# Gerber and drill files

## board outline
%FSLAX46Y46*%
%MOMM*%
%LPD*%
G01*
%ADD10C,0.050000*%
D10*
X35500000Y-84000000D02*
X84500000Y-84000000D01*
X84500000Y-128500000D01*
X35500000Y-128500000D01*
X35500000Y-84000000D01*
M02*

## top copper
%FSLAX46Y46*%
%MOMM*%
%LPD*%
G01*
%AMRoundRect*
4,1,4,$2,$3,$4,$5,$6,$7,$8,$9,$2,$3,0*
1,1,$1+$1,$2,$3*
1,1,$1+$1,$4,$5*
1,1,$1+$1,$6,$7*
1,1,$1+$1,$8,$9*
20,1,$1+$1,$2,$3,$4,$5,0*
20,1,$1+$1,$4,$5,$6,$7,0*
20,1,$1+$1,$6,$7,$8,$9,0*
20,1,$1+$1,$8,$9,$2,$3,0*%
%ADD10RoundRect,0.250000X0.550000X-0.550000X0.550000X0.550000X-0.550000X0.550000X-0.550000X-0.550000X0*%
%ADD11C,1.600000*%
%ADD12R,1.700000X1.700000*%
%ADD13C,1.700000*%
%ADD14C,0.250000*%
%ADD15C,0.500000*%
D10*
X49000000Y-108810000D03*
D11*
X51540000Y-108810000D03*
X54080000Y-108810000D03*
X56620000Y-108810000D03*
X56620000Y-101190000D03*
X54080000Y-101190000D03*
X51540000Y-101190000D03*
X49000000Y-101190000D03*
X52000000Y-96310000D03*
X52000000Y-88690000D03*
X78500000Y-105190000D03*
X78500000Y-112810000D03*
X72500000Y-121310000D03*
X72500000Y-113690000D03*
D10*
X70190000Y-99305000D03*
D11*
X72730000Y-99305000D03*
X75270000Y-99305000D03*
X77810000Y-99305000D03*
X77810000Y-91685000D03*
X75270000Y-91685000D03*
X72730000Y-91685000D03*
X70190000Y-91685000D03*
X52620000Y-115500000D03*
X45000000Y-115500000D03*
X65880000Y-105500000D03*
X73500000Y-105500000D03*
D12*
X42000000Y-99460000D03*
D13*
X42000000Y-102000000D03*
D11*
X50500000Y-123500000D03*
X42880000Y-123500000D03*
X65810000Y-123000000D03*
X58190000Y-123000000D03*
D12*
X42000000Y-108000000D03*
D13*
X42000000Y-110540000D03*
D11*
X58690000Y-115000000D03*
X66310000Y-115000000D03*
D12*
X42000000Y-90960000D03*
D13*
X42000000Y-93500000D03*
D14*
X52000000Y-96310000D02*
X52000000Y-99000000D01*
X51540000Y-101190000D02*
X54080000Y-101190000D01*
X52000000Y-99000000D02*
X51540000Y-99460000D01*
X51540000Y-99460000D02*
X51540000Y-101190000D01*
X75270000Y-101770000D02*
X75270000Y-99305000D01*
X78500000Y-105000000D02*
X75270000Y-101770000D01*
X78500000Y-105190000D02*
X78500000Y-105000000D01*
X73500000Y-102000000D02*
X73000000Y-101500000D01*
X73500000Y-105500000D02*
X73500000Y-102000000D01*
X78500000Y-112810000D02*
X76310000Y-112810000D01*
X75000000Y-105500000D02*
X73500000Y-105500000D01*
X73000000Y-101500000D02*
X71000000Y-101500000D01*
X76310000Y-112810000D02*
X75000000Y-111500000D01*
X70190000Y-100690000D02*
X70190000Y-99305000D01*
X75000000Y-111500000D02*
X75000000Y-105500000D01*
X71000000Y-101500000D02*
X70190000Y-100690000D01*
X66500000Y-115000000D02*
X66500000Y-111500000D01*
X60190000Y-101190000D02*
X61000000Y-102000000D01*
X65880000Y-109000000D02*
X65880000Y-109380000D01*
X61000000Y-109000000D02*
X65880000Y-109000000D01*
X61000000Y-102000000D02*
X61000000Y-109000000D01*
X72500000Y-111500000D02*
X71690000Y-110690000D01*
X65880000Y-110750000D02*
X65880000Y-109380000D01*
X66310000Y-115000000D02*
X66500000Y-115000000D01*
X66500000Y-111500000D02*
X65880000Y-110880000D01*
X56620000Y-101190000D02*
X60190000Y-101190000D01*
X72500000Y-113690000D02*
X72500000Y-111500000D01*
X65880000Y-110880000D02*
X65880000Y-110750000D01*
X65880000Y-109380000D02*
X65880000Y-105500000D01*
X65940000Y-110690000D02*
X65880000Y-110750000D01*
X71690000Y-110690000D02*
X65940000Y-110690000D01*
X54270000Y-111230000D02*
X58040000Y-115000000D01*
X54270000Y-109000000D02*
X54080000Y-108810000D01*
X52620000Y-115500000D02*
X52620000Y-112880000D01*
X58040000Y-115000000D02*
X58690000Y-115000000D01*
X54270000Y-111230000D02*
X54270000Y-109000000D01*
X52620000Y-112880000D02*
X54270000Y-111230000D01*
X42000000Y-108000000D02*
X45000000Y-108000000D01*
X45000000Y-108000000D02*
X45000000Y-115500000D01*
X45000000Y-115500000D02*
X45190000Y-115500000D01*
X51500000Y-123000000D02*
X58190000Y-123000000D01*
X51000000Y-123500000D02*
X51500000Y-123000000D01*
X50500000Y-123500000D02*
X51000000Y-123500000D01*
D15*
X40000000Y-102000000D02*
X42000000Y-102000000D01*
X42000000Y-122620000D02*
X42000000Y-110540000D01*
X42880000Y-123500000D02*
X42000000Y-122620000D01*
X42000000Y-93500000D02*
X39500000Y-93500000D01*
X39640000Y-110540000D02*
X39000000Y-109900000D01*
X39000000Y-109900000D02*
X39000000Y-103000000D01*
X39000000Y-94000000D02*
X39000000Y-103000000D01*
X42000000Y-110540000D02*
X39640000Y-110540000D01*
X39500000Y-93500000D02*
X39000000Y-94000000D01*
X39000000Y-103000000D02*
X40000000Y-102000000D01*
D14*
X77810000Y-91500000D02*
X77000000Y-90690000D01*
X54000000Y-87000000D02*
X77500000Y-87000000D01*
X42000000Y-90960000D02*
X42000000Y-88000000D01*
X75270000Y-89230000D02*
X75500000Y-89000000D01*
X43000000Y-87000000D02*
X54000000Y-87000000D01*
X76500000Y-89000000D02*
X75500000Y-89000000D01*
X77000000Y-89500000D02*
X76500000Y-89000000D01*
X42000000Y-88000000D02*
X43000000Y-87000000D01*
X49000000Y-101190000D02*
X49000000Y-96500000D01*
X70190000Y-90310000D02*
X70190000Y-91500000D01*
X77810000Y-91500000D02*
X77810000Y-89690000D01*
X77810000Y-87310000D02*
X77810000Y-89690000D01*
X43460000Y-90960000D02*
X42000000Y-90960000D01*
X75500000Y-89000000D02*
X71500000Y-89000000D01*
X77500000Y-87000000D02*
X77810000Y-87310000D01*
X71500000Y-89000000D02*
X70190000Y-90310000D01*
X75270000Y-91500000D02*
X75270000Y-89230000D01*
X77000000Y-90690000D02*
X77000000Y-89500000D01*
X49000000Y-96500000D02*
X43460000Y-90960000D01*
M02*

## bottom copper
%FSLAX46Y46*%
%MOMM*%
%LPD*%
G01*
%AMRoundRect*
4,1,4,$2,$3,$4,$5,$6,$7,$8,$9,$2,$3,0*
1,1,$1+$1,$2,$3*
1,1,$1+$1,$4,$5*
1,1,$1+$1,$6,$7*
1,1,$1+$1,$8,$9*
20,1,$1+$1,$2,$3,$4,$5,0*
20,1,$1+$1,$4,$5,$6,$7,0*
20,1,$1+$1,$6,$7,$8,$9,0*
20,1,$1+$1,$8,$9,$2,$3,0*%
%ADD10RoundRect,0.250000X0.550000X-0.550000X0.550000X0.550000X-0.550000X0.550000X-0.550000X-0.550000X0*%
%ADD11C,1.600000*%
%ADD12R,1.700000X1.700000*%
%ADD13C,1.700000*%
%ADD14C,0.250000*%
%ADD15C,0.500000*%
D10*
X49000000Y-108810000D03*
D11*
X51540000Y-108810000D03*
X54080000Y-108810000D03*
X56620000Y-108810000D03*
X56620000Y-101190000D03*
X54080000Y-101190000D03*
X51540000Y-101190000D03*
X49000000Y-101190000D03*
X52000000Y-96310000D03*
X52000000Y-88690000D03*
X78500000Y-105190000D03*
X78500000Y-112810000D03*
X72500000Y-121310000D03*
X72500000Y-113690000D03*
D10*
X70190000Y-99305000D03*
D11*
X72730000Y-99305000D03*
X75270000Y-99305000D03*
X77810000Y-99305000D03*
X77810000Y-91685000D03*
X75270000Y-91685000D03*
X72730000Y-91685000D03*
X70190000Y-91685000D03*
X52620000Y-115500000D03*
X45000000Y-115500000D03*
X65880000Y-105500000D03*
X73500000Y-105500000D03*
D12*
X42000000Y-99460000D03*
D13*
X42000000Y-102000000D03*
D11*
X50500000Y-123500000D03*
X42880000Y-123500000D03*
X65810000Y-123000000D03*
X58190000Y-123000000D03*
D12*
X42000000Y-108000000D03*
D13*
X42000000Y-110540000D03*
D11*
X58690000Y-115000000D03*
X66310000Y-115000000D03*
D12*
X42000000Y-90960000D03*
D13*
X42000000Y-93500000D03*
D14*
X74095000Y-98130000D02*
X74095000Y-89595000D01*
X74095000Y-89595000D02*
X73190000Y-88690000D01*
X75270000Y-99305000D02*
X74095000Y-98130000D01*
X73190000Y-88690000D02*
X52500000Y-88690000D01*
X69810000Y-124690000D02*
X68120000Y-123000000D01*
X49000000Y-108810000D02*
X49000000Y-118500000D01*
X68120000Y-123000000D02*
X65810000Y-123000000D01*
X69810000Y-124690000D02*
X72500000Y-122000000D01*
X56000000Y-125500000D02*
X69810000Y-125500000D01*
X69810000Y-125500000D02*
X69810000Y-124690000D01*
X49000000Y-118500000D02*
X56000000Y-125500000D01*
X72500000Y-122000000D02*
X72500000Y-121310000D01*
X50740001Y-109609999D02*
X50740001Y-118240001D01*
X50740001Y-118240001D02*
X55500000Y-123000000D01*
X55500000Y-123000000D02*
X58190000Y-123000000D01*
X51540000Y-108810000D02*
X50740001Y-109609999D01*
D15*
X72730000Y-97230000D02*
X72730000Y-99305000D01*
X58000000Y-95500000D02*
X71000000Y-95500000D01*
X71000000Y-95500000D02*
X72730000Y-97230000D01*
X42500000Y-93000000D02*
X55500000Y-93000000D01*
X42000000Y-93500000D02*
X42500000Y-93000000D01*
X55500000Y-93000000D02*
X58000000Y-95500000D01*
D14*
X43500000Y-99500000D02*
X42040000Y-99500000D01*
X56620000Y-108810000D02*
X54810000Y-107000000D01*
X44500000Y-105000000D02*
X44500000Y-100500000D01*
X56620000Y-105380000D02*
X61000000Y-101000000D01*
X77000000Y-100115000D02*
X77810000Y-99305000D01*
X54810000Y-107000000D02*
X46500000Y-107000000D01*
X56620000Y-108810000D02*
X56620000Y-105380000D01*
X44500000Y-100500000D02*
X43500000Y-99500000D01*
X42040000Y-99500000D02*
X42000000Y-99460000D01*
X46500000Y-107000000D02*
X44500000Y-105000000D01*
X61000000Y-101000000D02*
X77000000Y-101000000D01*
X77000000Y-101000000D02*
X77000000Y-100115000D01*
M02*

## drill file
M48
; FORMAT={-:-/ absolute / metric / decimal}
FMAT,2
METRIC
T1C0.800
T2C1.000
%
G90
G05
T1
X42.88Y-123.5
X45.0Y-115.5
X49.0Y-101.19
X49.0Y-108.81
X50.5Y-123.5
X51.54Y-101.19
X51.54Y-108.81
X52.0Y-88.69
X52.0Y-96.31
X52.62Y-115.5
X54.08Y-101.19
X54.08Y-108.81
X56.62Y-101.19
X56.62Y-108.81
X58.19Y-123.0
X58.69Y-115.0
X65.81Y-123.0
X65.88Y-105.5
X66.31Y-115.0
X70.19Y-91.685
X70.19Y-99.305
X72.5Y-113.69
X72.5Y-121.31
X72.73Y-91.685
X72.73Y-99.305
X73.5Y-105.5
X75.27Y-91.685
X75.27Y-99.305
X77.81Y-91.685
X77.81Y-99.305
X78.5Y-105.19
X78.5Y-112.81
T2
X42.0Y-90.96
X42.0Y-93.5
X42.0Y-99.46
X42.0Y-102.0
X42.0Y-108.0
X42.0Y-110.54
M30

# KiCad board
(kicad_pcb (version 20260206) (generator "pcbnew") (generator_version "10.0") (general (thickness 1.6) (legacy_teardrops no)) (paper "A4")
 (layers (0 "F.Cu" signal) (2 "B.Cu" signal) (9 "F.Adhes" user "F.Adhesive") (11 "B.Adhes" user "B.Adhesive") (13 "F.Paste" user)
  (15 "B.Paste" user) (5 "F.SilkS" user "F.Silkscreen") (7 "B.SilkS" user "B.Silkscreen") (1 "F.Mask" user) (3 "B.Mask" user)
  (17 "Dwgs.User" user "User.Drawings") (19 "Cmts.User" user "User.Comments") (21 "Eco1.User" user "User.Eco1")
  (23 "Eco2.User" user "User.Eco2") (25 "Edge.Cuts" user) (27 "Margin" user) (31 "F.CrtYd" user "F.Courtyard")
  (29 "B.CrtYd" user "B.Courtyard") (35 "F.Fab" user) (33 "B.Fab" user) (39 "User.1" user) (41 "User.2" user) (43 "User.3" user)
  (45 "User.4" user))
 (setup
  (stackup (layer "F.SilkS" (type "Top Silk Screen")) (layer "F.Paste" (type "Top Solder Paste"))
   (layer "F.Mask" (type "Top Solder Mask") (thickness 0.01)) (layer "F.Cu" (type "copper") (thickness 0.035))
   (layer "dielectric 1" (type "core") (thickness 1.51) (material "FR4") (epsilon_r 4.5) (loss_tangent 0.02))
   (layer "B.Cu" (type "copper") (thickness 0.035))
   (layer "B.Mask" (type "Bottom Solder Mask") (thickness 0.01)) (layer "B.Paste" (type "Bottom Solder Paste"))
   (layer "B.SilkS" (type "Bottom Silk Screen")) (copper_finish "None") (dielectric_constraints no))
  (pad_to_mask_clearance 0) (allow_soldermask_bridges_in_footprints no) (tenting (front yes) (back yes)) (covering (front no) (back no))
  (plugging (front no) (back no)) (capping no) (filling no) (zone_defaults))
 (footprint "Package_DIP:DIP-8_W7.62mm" (layer "F.Cu") (at 49 108.81 90)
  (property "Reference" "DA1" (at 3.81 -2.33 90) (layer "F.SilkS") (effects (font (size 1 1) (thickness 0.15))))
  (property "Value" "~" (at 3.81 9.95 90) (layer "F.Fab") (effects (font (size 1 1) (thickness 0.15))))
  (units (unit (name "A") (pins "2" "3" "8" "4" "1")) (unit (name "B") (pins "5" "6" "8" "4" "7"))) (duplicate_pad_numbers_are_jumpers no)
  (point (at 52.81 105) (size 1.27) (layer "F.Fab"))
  (pad "1" thru_hole roundrect (at 0 0 90) (size 1.6 1.6) (drill 0.8) (layers "*.Cu" "*.Mask") (remove_unused_layers no)
   (roundrect_rratio 0.15625) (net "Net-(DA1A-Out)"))
  (pad "2" thru_hole circle (at 0 2.54 90) (size 1.6 1.6) (drill 0.8) (layers "*.Cu" "*.Mask") (remove_unused_layers no)
   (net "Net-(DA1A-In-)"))
  (pad "3" thru_hole circle (at 0 5.08 90) (size 1.6 1.6) (drill 0.8) (layers "*.Cu" "*.Mask") (remove_unused_layers no)
   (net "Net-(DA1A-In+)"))
  (pad "4" thru_hole circle (at 0 7.62 90) (size 1.6 1.6) (drill 0.8) (layers "*.Cu" "*.Mask") (remove_unused_layers no) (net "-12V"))
  (pad "5" thru_hole circle (at 7.62 7.62 90) (size 1.6 1.6) (drill 0.8) (layers "*.Cu" "*.Mask") (remove_unused_layers no)
   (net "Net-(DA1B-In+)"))
  (pad "6" thru_hole circle (at 7.62 5.08 90) (size 1.6 1.6) (drill 0.8) (layers "*.Cu" "*.Mask") (remove_unused_layers no)
   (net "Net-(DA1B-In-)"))
  (pad "7" thru_hole circle (at 7.62 2.54 90) (size 1.6 1.6) (drill 0.8) (layers "*.Cu" "*.Mask") (remove_unused_layers no)
   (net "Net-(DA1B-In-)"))
  (pad "8" thru_hole circle (at 7.62 0 90) (size 1.6 1.6) (drill 0.8) (layers "*.Cu" "*.Mask") (remove_unused_layers no) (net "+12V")))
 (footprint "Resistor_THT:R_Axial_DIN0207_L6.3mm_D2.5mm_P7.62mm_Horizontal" (layer "F.Cu") (at 52 96.31 90)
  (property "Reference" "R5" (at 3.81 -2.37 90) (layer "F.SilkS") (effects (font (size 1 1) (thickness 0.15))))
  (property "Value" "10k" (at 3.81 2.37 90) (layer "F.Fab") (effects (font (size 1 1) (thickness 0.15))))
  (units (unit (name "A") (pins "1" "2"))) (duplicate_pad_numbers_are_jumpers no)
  (pad "1" thru_hole circle (at 0 0 90) (size 1.6 1.6) (drill 0.8) (layers "*.Cu" "*.Mask") (remove_unused_layers no) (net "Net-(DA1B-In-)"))
  (pad "2" thru_hole circle (at 7.62 0 90) (size 1.6 1.6) (drill 0.8) (layers "*.Cu" "*.Mask") (remove_unused_layers no)
   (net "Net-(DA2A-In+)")))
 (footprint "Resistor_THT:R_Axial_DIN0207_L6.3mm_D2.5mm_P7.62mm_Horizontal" (layer "F.Cu") (at 78.5 105.19 -90)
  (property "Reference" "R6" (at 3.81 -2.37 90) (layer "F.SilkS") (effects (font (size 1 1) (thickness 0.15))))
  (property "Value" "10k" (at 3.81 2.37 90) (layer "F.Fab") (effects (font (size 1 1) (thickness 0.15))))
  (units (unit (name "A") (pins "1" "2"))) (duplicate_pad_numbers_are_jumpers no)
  (pad "1" thru_hole circle (at 0 0 270) (size 1.6 1.6) (drill 0.8) (layers "*.Cu" "*.Mask") (remove_unused_layers no)
   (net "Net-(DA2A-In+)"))
  (pad "2" thru_hole circle (at 7.62 0 270) (size 1.6 1.6) (drill 0.8) (layers "*.Cu" "*.Mask") (remove_unused_layers no)
   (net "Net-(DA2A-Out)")))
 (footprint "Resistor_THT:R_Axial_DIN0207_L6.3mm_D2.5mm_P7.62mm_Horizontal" (layer "F.Cu") (at 72.5 121.31 90)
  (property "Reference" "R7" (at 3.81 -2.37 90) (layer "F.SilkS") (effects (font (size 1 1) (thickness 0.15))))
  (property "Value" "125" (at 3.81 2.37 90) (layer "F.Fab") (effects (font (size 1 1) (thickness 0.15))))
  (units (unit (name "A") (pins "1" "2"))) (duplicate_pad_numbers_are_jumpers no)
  (pad "1" thru_hole circle (at 0 0 90) (size 1.6 1.6) (drill 0.8) (layers "*.Cu" "*.Mask") (remove_unused_layers no) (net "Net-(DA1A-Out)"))
  (pad "2" thru_hole circle (at 7.62 0 90) (size 1.6 1.6) (drill 0.8) (layers "*.Cu" "*.Mask") (remove_unused_layers no)
   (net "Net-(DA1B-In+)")))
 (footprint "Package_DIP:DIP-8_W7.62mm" (layer "F.Cu") (at 70.19 99.305 90)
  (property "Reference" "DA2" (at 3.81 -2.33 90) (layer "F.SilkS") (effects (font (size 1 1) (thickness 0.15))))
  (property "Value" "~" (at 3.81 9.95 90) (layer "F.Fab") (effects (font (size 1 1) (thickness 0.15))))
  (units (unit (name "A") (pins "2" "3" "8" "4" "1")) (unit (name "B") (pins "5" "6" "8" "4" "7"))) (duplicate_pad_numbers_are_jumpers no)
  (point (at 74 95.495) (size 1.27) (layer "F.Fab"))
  (pad "1" thru_hole roundrect (at 0 0 90) (size 1.6 1.6) (drill 0.8) (layers "*.Cu" "*.Mask") (remove_unused_layers no)
   (roundrect_rratio 0.15625) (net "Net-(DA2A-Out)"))
  (pad "2" thru_hole circle (at 0 2.54 90) (size 1.6 1.6) (drill 0.8) (layers "*.Cu" "*.Mask") (remove_unused_layers no) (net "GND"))
  (pad "3" thru_hole circle (at 0 5.08 90) (size 1.6 1.6) (drill 0.8) (layers "*.Cu" "*.Mask") (remove_unused_layers no)
   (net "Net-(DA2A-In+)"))
  (pad "4" thru_hole circle (at 0 7.62 90) (size 1.6 1.6) (drill 0.8) (layers "*.Cu" "*.Mask") (remove_unused_layers no) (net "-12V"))
  (pad "5" thru_hole circle (at 7.62 7.62 90) (size 1.6 1.6) (drill 0.8) (layers "*.Cu" "*.Mask") (remove_unused_layers no) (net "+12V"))
  (pad "6" thru_hole circle (at 7.62 5.08 90) (size 1.6 1.6) (drill 0.8) (layers "*.Cu" "*.Mask") (remove_unused_layers no) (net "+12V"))
  (pad "7" thru_hole circle (at 7.62 2.54 90) (size 1.6 1.6) (drill 0.8) (layers "*.Cu" "*.Mask") (remove_unused_layers no)
   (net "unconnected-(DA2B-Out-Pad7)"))
  (pad "8" thru_hole circle (at 7.62 0 90) (size 1.6 1.6) (drill 0.8) (layers "*.Cu" "*.Mask") (remove_unused_layers no) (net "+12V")))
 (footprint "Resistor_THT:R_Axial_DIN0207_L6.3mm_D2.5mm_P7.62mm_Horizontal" (layer "F.Cu") (at 52.62 115.5 180)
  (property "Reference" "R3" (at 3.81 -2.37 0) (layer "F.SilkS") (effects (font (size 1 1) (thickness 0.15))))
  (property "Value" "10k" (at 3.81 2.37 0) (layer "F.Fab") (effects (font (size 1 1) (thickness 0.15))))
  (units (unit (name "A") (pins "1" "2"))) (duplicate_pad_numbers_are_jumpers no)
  (pad "1" thru_hole circle (at 0 0 180) (size 1.6 1.6) (drill 0.8) (layers "*.Cu" "*.Mask") (remove_unused_layers no)
   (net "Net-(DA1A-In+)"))
  (pad "2" thru_hole circle (at 7.62 0 180) (size 1.6 1.6) (drill 0.8) (layers "*.Cu" "*.Mask") (remove_unused_layers no)
   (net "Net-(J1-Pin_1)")))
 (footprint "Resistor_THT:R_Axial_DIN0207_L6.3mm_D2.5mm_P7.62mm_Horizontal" (layer "F.Cu") (at 65.88 105.5)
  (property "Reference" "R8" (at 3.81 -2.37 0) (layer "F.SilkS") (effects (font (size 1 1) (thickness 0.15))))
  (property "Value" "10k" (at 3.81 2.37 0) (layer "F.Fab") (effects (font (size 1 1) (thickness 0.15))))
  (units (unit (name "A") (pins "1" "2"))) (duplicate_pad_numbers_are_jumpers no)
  (pad "1" thru_hole circle (at 0 0) (size 1.6 1.6) (drill 0.8) (layers "*.Cu" "*.Mask") (remove_unused_layers no) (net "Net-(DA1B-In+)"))
  (pad "2" thru_hole circle (at 7.62 0) (size 1.6 1.6) (drill 0.8) (layers "*.Cu" "*.Mask") (remove_unused_layers no) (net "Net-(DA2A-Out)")))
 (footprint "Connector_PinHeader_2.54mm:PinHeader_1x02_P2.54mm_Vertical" (layer "F.Cu") (at 42 99.46)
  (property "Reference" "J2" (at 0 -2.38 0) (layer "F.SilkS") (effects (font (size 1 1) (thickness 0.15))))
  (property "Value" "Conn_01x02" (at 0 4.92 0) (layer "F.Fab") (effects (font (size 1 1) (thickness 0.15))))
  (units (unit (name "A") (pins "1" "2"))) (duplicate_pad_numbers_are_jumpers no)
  (pad "1" thru_hole rect (at 0 0) (size 1.7 1.7) (drill 1) (layers "*.Cu" "*.Mask") (remove_unused_layers no) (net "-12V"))
  (pad "2" thru_hole circle (at 0 2.54) (size 1.7 1.7) (drill 1) (layers "*.Cu" "*.Mask") (remove_unused_layers no) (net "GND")))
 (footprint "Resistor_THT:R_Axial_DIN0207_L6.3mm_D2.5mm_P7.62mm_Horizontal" (layer "F.Cu") (at 50.5 123.5 180)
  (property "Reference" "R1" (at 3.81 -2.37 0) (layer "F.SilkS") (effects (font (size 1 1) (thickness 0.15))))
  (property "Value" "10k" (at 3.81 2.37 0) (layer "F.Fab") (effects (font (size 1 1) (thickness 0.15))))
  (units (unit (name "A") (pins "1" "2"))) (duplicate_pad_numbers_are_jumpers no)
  (pad "1" thru_hole circle (at 0 0 180) (size 1.6 1.6) (drill 0.8) (layers "*.Cu" "*.Mask") (remove_unused_layers no)
   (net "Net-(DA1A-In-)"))
  (pad "2" thru_hole circle (at 7.62 0 180) (size 1.6 1.6) (drill 0.8) (layers "*.Cu" "*.Mask") (remove_unused_layers no) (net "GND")))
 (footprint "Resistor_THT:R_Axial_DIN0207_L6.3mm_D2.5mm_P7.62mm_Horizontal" (layer "F.Cu") (at 65.81 123 180)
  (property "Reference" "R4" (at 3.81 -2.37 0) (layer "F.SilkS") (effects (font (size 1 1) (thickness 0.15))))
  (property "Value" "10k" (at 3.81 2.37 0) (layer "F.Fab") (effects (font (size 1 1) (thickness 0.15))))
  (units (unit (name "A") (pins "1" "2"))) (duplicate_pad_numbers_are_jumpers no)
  (pad "1" thru_hole circle (at 0 0 180) (size 1.6 1.6) (drill 0.8) (layers "*.Cu" "*.Mask") (remove_unused_layers no)
   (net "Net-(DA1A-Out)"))
  (pad "2" thru_hole circle (at 7.62 0 180) (size 1.6 1.6) (drill 0.8) (layers "*.Cu" "*.Mask") (remove_unused_layers no)
   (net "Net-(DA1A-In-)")))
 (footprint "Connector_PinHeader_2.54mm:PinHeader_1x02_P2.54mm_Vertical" (layer "F.Cu") (at 42 108)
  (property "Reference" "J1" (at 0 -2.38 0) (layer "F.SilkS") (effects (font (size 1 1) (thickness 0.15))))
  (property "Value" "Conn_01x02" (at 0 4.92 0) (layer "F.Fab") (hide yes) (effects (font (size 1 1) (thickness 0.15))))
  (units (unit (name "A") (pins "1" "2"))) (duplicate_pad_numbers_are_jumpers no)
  (pad "1" thru_hole rect (at 0 0) (size 1.7 1.7) (drill 1) (layers "*.Cu" "*.Mask") (remove_unused_layers no) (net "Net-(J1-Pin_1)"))
  (pad "2" thru_hole circle (at 0 2.54) (size 1.7 1.7) (drill 1) (layers "*.Cu" "*.Mask") (remove_unused_layers no) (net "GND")))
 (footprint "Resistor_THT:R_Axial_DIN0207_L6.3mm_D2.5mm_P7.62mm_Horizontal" (layer "F.Cu") (at 58.69 115)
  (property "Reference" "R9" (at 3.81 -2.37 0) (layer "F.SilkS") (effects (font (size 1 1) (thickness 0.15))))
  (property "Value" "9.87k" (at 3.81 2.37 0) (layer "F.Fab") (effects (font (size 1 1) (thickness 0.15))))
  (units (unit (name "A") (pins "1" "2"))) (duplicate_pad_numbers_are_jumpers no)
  (pad "1" thru_hole circle (at 0 0) (size 1.6 1.6) (drill 0.8) (layers "*.Cu" "*.Mask") (remove_unused_layers no) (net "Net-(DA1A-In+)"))
  (pad "2" thru_hole circle (at 7.62 0) (size 1.6 1.6) (drill 0.8) (layers "*.Cu" "*.Mask") (remove_unused_layers no) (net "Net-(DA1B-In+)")))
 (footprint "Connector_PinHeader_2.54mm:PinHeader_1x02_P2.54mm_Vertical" (layer "F.Cu") (at 42 90.96)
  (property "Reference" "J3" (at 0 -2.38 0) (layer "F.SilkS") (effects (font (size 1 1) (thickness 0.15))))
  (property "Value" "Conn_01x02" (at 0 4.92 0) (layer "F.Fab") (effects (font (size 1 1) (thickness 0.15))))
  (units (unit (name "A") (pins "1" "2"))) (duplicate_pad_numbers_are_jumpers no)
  (pad "1" thru_hole rect (at 0 0) (size 1.7 1.7) (drill 1) (layers "*.Cu" "*.Mask") (remove_unused_layers no) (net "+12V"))
  (pad "2" thru_hole circle (at 0 2.54) (size 1.7 1.7) (drill 1) (layers "*.Cu" "*.Mask") (remove_unused_layers no) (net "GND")))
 (gr_rect (start 35.5 84) (end 84.5 128.5) (stroke (width 0.05) (type default)) (fill no) (layer "Edge.Cuts"))
 (segment (start 52 96.31) (end 52 99) (width 0.25) (layer "F.Cu") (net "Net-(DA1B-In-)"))
 (segment (start 51.54 101.19) (end 54.08 101.19) (width 0.25) (layer "F.Cu") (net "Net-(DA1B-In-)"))
 (segment (start 52 99) (end 51.54 99.46) (width 0.25) (layer "F.Cu") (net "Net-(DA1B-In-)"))
 (segment (start 51.54 99.46) (end 51.54 101.19) (width 0.25) (layer "F.Cu") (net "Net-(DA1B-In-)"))
 (segment (start 75.27 101.77) (end 75.27 99.305) (width 0.25) (layer "F.Cu") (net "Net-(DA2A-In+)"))
 (segment (start 78.5 105) (end 75.27 101.77) (width 0.25) (layer "F.Cu") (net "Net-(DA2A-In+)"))
 (segment (start 78.5 105.19) (end 78.5 105) (width 0.25) (layer "F.Cu") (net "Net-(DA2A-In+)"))
 (segment (start 74.095 98.13) (end 74.095 89.595) (width 0.25) (layer "B.Cu") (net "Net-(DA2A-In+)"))
 (segment (start 74.095 89.595) (end 73.19 88.69) (width 0.25) (layer "B.Cu") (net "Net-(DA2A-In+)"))
 (segment (start 75.27 99.305) (end 74.095 98.13) (width 0.25) (layer "B.Cu") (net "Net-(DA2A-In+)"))
 (segment (start 73.19 88.69) (end 52.5 88.69) (width 0.25) (layer "B.Cu") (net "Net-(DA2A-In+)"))
 (segment (start 73.5 102) (end 73 101.5) (width 0.25) (layer "F.Cu") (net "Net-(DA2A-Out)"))
 (segment (start 73.5 105.5) (end 73.5 102) (width 0.25) (layer "F.Cu") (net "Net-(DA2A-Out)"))
 (segment (start 78.5 112.81) (end 76.31 112.81) (width 0.25) (layer "F.Cu") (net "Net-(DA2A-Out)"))
 (segment (start 75 105.5) (end 73.5 105.5) (width 0.25) (layer "F.Cu") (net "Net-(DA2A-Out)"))
 (segment (start 73 101.5) (end 71 101.5) (width 0.25) (layer "F.Cu") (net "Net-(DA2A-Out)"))
 (segment (start 76.31 112.81) (end 75 111.5) (width 0.25) (layer "F.Cu") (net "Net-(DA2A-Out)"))
 (segment (start 70.19 100.69) (end 70.19 99.305) (width 0.25) (layer "F.Cu") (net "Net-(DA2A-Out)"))
 (segment (start 75 111.5) (end 75 105.5) (width 0.25) (layer "F.Cu") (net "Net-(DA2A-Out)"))
 (segment (start 71 101.5) (end 70.19 100.69) (width 0.25) (layer "F.Cu") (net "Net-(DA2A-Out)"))
 (segment (start 69.81 124.69) (end 68.12 123) (width 0.25) (layer "B.Cu") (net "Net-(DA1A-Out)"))
 (segment (start 49 108.81) (end 49 118.5) (width 0.25) (layer "B.Cu") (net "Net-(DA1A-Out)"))
 (segment (start 68.12 123) (end 65.81 123) (width 0.25) (layer "B.Cu") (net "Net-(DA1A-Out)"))
 (segment (start 69.81 124.69) (end 72.5 122) (width 0.25) (layer "B.Cu") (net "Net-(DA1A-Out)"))
 (segment (start 56 125.5) (end 69.81 125.5) (width 0.25) (layer "B.Cu") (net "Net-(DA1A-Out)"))
 (segment (start 69.81 125.5) (end 69.81 124.69) (width 0.25) (layer "B.Cu") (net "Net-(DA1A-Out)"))
 (segment (start 49 118.5) (end 56 125.5) (width 0.25) (layer "B.Cu") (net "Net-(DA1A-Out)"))
 (segment (start 72.5 122) (end 72.5 121.31) (width 0.25) (layer "B.Cu") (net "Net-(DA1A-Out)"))
 (segment (start 66.5 115) (end 66.5 111.5) (width 0.25) (layer "F.Cu") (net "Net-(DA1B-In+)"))
 (segment (start 60.19 101.19) (end 61 102) (width 0.25) (layer "F.Cu") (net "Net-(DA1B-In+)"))
 (segment (start 65.88 109) (end 65.88 109.38) (width 0.25) (layer "F.Cu") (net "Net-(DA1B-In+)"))
 (segment (start 61 109) (end 65.88 109) (width 0.25) (layer "F.Cu") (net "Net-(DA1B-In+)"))
 (segment (start 61 102) (end 61 109) (width 0.25) (layer "F.Cu") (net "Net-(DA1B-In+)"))
 (segment (start 72.5 111.5) (end 71.69 110.69) (width 0.25) (layer "F.Cu") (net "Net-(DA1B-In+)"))
 (segment (start 65.88 110.75) (end 65.88 109.38) (width 0.25) (layer "F.Cu") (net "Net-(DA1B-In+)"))
 (segment (start 66.31 115) (end 66.5 115) (width 0.25) (layer "F.Cu") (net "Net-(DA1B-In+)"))
 (segment (start 66.5 111.5) (end 65.88 110.88) (width 0.25) (layer "F.Cu") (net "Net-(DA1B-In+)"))
 (segment (start 56.62 101.19) (end 60.19 101.19) (width 0.25) (layer "F.Cu") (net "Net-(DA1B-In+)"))
 (segment (start 72.5 113.69) (end 72.5 111.5) (width 0.25) (layer "F.Cu") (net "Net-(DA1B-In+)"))
 (segment (start 65.88 110.88) (end 65.88 110.75) (width 0.25) (layer "F.Cu") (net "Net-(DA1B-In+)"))
 (segment (start 65.88 109.38) (end 65.88 105.5) (width 0.25) (layer "F.Cu") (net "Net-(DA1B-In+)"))
 (segment (start 65.94 110.69) (end 65.88 110.75) (width 0.25) (layer "F.Cu") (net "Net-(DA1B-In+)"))
 (segment (start 71.69 110.69) (end 65.94 110.69) (width 0.25) (layer "F.Cu") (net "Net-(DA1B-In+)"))
 (segment (start 54.27 111.23) (end 58.04 115) (width 0.25) (layer "F.Cu") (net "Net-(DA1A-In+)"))
 (segment (start 54.27 109) (end 54.08 108.81) (width 0.25) (layer "F.Cu") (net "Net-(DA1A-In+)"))
 (segment (start 52.62 115.5) (end 52.62 112.88) (width 0.25) (layer "F.Cu") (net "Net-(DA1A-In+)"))
 (segment (start 58.04 115) (end 58.69 115) (width 0.25) (layer "F.Cu") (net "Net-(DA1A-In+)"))
 (segment (start 54.27 111.23) (end 54.27 109) (width 0.25) (layer "F.Cu") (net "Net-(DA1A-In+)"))
 (segment (start 52.62 112.88) (end 54.27 111.23) (width 0.25) (layer "F.Cu") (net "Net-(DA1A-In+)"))
 (segment (start 42 108) (end 45 108) (width 0.25) (layer "F.Cu") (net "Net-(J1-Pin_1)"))
 (segment (start 45 108) (end 45 115.5) (width 0.25) (layer "F.Cu") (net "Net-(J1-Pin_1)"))
 (segment (start 45 115.5) (end 45.19 115.5) (width 0.25) (layer "F.Cu") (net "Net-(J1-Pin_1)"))
 (segment (start 51.5 123) (end 58.19 123) (width 0.25) (layer "F.Cu") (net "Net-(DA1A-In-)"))
 (segment (start 51 123.5) (end 51.5 123) (width 0.25) (layer "F.Cu") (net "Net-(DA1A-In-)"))
 (segment (start 50.5 123.5) (end 51 123.5) (width 0.25) (layer "F.Cu") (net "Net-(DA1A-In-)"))
 (segment (start 50.740001 109.609999) (end 50.740001 118.240001) (width 0.25) (layer "B.Cu") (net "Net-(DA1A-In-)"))
 (segment (start 50.740001 118.240001) (end 55.5 123) (width 0.25) (layer "B.Cu") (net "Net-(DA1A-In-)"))
 (segment (start 55.5 123) (end 58.19 123) (width 0.25) (layer "B.Cu") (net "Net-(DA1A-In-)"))
 (segment (start 51.54 108.81) (end 50.740001 109.609999) (width 0.25) (layer "B.Cu") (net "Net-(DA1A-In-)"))
 (segment (start 40 102) (end 42 102) (width 0.5) (layer "F.Cu") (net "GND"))
 (segment (start 42 122.62) (end 42 110.54) (width 0.5) (layer "F.Cu") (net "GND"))
 (segment (start 42.88 123.5) (end 42 122.62) (width 0.5) (layer "F.Cu") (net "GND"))
 (segment (start 42 93.5) (end 39.5 93.5) (width 0.5) (layer "F.Cu") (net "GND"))
 (segment (start 39.64 110.54) (end 39 109.9) (width 0.5) (layer "F.Cu") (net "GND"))
 (segment (start 39 109.9) (end 39 103) (width 0.5) (layer "F.Cu") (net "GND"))
 (segment (start 39 94) (end 39 103) (width 0.5) (layer "F.Cu") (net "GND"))
 (segment (start 42 110.54) (end 39.64 110.54) (width 0.5) (layer "F.Cu") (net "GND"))
 (segment (start 39.5 93.5) (end 39 94) (width 0.5) (layer "F.Cu") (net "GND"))
 (segment (start 39 103) (end 40 102) (width 0.5) (layer "F.Cu") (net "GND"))
 (segment (start 72.73 97.23) (end 72.73 99.305) (width 0.5) (layer "B.Cu") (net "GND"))
 (segment (start 58 95.5) (end 71 95.5) (width 0.5) (layer "B.Cu") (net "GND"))
 (segment (start 71 95.5) (end 72.73 97.23) (width 0.5) (layer "B.Cu") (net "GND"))
 (segment (start 42.5 93) (end 55.5 93) (width 0.5) (layer "B.Cu") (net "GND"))
 (segment (start 42 93.5) (end 42.5 93) (width 0.5) (layer "B.Cu") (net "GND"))
 (segment (start 55.5 93) (end 58 95.5) (width 0.5) (layer "B.Cu") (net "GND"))
 (segment (start 77.81 91.5) (end 77 90.69) (width 0.25) (layer "F.Cu") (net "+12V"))
 (segment (start 54 87) (end 77.5 87) (width 0.25) (layer "F.Cu") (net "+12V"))
 (segment (start 42 90.96) (end 42 88) (width 0.25) (layer "F.Cu") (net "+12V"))
 (segment (start 75.27 89.23) (end 75.5 89) (width 0.25) (layer "F.Cu") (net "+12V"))
 (segment (start 43 87) (end 54 87) (width 0.25) (layer "F.Cu") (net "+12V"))
 (segment (start 76.5 89) (end 75.5 89) (width 0.25) (layer "F.Cu") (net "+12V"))
 (segment (start 77 89.5) (end 76.5 89) (width 0.25) (layer "F.Cu") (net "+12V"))
 (segment (start 42 88) (end 43 87) (width 0.25) (layer "F.Cu") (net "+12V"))
 (segment (start 49 101.19) (end 49 96.5) (width 0.25) (layer "F.Cu") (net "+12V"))
 (segment (start 70.19 90.31) (end 70.19 91.5) (width 0.25) (layer "F.Cu") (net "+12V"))
 (segment (start 77.81 91.5) (end 77.81 89.69) (width 0.25) (layer "F.Cu") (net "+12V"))
 (segment (start 77.81 87.31) (end 77.81 89.69) (width 0.25) (layer "F.Cu") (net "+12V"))
 (segment (start 43.46 90.96) (end 42 90.96) (width 0.25) (layer "F.Cu") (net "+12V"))
 (segment (start 75.5 89) (end 71.5 89) (width 0.25) (layer "F.Cu") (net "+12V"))
 (segment (start 77.5 87) (end 77.81 87.31) (width 0.25) (layer "F.Cu") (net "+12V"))
 (segment (start 71.5 89) (end 70.19 90.31) (width 0.25) (layer "F.Cu") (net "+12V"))
 (segment (start 75.27 91.5) (end 75.27 89.23) (width 0.25) (layer "F.Cu") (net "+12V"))
 (segment (start 77 90.69) (end 77 89.5) (width 0.25) (layer "F.Cu") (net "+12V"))
 (segment (start 49 96.5) (end 43.46 90.96) (width 0.25) (layer "F.Cu") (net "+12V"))
 (segment (start 43.5 99.5) (end 42.04 99.5) (width 0.25) (layer "B.Cu") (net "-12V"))
 (segment (start 56.62 108.81) (end 54.81 107) (width 0.25) (layer "B.Cu") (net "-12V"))
 (segment (start 44.5 105) (end 44.5 100.5) (width 0.25) (layer "B.Cu") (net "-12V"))
 (segment (start 56.62 105.38) (end 61 101) (width 0.25) (layer "B.Cu") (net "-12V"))
 (segment (start 77 100.115) (end 77.81 99.305) (width 0.25) (layer "B.Cu") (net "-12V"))
 (segment (start 54.81 107) (end 46.5 107) (width 0.25) (layer "B.Cu") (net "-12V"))
 (segment (start 56.62 108.81) (end 56.62 105.38) (width 0.25) (layer "B.Cu") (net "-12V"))
 (segment (start 44.5 100.5) (end 43.5 99.5) (width 0.25) (layer "B.Cu") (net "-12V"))
 (segment (start 42.04 99.5) (end 42 99.46) (width 0.25) (layer "B.Cu") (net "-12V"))
 (segment (start 46.5 107) (end 44.5 105) (width 0.25) (layer "B.Cu") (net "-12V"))
 (segment (start 61 101) (end 77 101) (width 0.25) (layer "B.Cu") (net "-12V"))
 (segment (start 77 101) (end 77 100.115) (width 0.25) (layer "B.Cu") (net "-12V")))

